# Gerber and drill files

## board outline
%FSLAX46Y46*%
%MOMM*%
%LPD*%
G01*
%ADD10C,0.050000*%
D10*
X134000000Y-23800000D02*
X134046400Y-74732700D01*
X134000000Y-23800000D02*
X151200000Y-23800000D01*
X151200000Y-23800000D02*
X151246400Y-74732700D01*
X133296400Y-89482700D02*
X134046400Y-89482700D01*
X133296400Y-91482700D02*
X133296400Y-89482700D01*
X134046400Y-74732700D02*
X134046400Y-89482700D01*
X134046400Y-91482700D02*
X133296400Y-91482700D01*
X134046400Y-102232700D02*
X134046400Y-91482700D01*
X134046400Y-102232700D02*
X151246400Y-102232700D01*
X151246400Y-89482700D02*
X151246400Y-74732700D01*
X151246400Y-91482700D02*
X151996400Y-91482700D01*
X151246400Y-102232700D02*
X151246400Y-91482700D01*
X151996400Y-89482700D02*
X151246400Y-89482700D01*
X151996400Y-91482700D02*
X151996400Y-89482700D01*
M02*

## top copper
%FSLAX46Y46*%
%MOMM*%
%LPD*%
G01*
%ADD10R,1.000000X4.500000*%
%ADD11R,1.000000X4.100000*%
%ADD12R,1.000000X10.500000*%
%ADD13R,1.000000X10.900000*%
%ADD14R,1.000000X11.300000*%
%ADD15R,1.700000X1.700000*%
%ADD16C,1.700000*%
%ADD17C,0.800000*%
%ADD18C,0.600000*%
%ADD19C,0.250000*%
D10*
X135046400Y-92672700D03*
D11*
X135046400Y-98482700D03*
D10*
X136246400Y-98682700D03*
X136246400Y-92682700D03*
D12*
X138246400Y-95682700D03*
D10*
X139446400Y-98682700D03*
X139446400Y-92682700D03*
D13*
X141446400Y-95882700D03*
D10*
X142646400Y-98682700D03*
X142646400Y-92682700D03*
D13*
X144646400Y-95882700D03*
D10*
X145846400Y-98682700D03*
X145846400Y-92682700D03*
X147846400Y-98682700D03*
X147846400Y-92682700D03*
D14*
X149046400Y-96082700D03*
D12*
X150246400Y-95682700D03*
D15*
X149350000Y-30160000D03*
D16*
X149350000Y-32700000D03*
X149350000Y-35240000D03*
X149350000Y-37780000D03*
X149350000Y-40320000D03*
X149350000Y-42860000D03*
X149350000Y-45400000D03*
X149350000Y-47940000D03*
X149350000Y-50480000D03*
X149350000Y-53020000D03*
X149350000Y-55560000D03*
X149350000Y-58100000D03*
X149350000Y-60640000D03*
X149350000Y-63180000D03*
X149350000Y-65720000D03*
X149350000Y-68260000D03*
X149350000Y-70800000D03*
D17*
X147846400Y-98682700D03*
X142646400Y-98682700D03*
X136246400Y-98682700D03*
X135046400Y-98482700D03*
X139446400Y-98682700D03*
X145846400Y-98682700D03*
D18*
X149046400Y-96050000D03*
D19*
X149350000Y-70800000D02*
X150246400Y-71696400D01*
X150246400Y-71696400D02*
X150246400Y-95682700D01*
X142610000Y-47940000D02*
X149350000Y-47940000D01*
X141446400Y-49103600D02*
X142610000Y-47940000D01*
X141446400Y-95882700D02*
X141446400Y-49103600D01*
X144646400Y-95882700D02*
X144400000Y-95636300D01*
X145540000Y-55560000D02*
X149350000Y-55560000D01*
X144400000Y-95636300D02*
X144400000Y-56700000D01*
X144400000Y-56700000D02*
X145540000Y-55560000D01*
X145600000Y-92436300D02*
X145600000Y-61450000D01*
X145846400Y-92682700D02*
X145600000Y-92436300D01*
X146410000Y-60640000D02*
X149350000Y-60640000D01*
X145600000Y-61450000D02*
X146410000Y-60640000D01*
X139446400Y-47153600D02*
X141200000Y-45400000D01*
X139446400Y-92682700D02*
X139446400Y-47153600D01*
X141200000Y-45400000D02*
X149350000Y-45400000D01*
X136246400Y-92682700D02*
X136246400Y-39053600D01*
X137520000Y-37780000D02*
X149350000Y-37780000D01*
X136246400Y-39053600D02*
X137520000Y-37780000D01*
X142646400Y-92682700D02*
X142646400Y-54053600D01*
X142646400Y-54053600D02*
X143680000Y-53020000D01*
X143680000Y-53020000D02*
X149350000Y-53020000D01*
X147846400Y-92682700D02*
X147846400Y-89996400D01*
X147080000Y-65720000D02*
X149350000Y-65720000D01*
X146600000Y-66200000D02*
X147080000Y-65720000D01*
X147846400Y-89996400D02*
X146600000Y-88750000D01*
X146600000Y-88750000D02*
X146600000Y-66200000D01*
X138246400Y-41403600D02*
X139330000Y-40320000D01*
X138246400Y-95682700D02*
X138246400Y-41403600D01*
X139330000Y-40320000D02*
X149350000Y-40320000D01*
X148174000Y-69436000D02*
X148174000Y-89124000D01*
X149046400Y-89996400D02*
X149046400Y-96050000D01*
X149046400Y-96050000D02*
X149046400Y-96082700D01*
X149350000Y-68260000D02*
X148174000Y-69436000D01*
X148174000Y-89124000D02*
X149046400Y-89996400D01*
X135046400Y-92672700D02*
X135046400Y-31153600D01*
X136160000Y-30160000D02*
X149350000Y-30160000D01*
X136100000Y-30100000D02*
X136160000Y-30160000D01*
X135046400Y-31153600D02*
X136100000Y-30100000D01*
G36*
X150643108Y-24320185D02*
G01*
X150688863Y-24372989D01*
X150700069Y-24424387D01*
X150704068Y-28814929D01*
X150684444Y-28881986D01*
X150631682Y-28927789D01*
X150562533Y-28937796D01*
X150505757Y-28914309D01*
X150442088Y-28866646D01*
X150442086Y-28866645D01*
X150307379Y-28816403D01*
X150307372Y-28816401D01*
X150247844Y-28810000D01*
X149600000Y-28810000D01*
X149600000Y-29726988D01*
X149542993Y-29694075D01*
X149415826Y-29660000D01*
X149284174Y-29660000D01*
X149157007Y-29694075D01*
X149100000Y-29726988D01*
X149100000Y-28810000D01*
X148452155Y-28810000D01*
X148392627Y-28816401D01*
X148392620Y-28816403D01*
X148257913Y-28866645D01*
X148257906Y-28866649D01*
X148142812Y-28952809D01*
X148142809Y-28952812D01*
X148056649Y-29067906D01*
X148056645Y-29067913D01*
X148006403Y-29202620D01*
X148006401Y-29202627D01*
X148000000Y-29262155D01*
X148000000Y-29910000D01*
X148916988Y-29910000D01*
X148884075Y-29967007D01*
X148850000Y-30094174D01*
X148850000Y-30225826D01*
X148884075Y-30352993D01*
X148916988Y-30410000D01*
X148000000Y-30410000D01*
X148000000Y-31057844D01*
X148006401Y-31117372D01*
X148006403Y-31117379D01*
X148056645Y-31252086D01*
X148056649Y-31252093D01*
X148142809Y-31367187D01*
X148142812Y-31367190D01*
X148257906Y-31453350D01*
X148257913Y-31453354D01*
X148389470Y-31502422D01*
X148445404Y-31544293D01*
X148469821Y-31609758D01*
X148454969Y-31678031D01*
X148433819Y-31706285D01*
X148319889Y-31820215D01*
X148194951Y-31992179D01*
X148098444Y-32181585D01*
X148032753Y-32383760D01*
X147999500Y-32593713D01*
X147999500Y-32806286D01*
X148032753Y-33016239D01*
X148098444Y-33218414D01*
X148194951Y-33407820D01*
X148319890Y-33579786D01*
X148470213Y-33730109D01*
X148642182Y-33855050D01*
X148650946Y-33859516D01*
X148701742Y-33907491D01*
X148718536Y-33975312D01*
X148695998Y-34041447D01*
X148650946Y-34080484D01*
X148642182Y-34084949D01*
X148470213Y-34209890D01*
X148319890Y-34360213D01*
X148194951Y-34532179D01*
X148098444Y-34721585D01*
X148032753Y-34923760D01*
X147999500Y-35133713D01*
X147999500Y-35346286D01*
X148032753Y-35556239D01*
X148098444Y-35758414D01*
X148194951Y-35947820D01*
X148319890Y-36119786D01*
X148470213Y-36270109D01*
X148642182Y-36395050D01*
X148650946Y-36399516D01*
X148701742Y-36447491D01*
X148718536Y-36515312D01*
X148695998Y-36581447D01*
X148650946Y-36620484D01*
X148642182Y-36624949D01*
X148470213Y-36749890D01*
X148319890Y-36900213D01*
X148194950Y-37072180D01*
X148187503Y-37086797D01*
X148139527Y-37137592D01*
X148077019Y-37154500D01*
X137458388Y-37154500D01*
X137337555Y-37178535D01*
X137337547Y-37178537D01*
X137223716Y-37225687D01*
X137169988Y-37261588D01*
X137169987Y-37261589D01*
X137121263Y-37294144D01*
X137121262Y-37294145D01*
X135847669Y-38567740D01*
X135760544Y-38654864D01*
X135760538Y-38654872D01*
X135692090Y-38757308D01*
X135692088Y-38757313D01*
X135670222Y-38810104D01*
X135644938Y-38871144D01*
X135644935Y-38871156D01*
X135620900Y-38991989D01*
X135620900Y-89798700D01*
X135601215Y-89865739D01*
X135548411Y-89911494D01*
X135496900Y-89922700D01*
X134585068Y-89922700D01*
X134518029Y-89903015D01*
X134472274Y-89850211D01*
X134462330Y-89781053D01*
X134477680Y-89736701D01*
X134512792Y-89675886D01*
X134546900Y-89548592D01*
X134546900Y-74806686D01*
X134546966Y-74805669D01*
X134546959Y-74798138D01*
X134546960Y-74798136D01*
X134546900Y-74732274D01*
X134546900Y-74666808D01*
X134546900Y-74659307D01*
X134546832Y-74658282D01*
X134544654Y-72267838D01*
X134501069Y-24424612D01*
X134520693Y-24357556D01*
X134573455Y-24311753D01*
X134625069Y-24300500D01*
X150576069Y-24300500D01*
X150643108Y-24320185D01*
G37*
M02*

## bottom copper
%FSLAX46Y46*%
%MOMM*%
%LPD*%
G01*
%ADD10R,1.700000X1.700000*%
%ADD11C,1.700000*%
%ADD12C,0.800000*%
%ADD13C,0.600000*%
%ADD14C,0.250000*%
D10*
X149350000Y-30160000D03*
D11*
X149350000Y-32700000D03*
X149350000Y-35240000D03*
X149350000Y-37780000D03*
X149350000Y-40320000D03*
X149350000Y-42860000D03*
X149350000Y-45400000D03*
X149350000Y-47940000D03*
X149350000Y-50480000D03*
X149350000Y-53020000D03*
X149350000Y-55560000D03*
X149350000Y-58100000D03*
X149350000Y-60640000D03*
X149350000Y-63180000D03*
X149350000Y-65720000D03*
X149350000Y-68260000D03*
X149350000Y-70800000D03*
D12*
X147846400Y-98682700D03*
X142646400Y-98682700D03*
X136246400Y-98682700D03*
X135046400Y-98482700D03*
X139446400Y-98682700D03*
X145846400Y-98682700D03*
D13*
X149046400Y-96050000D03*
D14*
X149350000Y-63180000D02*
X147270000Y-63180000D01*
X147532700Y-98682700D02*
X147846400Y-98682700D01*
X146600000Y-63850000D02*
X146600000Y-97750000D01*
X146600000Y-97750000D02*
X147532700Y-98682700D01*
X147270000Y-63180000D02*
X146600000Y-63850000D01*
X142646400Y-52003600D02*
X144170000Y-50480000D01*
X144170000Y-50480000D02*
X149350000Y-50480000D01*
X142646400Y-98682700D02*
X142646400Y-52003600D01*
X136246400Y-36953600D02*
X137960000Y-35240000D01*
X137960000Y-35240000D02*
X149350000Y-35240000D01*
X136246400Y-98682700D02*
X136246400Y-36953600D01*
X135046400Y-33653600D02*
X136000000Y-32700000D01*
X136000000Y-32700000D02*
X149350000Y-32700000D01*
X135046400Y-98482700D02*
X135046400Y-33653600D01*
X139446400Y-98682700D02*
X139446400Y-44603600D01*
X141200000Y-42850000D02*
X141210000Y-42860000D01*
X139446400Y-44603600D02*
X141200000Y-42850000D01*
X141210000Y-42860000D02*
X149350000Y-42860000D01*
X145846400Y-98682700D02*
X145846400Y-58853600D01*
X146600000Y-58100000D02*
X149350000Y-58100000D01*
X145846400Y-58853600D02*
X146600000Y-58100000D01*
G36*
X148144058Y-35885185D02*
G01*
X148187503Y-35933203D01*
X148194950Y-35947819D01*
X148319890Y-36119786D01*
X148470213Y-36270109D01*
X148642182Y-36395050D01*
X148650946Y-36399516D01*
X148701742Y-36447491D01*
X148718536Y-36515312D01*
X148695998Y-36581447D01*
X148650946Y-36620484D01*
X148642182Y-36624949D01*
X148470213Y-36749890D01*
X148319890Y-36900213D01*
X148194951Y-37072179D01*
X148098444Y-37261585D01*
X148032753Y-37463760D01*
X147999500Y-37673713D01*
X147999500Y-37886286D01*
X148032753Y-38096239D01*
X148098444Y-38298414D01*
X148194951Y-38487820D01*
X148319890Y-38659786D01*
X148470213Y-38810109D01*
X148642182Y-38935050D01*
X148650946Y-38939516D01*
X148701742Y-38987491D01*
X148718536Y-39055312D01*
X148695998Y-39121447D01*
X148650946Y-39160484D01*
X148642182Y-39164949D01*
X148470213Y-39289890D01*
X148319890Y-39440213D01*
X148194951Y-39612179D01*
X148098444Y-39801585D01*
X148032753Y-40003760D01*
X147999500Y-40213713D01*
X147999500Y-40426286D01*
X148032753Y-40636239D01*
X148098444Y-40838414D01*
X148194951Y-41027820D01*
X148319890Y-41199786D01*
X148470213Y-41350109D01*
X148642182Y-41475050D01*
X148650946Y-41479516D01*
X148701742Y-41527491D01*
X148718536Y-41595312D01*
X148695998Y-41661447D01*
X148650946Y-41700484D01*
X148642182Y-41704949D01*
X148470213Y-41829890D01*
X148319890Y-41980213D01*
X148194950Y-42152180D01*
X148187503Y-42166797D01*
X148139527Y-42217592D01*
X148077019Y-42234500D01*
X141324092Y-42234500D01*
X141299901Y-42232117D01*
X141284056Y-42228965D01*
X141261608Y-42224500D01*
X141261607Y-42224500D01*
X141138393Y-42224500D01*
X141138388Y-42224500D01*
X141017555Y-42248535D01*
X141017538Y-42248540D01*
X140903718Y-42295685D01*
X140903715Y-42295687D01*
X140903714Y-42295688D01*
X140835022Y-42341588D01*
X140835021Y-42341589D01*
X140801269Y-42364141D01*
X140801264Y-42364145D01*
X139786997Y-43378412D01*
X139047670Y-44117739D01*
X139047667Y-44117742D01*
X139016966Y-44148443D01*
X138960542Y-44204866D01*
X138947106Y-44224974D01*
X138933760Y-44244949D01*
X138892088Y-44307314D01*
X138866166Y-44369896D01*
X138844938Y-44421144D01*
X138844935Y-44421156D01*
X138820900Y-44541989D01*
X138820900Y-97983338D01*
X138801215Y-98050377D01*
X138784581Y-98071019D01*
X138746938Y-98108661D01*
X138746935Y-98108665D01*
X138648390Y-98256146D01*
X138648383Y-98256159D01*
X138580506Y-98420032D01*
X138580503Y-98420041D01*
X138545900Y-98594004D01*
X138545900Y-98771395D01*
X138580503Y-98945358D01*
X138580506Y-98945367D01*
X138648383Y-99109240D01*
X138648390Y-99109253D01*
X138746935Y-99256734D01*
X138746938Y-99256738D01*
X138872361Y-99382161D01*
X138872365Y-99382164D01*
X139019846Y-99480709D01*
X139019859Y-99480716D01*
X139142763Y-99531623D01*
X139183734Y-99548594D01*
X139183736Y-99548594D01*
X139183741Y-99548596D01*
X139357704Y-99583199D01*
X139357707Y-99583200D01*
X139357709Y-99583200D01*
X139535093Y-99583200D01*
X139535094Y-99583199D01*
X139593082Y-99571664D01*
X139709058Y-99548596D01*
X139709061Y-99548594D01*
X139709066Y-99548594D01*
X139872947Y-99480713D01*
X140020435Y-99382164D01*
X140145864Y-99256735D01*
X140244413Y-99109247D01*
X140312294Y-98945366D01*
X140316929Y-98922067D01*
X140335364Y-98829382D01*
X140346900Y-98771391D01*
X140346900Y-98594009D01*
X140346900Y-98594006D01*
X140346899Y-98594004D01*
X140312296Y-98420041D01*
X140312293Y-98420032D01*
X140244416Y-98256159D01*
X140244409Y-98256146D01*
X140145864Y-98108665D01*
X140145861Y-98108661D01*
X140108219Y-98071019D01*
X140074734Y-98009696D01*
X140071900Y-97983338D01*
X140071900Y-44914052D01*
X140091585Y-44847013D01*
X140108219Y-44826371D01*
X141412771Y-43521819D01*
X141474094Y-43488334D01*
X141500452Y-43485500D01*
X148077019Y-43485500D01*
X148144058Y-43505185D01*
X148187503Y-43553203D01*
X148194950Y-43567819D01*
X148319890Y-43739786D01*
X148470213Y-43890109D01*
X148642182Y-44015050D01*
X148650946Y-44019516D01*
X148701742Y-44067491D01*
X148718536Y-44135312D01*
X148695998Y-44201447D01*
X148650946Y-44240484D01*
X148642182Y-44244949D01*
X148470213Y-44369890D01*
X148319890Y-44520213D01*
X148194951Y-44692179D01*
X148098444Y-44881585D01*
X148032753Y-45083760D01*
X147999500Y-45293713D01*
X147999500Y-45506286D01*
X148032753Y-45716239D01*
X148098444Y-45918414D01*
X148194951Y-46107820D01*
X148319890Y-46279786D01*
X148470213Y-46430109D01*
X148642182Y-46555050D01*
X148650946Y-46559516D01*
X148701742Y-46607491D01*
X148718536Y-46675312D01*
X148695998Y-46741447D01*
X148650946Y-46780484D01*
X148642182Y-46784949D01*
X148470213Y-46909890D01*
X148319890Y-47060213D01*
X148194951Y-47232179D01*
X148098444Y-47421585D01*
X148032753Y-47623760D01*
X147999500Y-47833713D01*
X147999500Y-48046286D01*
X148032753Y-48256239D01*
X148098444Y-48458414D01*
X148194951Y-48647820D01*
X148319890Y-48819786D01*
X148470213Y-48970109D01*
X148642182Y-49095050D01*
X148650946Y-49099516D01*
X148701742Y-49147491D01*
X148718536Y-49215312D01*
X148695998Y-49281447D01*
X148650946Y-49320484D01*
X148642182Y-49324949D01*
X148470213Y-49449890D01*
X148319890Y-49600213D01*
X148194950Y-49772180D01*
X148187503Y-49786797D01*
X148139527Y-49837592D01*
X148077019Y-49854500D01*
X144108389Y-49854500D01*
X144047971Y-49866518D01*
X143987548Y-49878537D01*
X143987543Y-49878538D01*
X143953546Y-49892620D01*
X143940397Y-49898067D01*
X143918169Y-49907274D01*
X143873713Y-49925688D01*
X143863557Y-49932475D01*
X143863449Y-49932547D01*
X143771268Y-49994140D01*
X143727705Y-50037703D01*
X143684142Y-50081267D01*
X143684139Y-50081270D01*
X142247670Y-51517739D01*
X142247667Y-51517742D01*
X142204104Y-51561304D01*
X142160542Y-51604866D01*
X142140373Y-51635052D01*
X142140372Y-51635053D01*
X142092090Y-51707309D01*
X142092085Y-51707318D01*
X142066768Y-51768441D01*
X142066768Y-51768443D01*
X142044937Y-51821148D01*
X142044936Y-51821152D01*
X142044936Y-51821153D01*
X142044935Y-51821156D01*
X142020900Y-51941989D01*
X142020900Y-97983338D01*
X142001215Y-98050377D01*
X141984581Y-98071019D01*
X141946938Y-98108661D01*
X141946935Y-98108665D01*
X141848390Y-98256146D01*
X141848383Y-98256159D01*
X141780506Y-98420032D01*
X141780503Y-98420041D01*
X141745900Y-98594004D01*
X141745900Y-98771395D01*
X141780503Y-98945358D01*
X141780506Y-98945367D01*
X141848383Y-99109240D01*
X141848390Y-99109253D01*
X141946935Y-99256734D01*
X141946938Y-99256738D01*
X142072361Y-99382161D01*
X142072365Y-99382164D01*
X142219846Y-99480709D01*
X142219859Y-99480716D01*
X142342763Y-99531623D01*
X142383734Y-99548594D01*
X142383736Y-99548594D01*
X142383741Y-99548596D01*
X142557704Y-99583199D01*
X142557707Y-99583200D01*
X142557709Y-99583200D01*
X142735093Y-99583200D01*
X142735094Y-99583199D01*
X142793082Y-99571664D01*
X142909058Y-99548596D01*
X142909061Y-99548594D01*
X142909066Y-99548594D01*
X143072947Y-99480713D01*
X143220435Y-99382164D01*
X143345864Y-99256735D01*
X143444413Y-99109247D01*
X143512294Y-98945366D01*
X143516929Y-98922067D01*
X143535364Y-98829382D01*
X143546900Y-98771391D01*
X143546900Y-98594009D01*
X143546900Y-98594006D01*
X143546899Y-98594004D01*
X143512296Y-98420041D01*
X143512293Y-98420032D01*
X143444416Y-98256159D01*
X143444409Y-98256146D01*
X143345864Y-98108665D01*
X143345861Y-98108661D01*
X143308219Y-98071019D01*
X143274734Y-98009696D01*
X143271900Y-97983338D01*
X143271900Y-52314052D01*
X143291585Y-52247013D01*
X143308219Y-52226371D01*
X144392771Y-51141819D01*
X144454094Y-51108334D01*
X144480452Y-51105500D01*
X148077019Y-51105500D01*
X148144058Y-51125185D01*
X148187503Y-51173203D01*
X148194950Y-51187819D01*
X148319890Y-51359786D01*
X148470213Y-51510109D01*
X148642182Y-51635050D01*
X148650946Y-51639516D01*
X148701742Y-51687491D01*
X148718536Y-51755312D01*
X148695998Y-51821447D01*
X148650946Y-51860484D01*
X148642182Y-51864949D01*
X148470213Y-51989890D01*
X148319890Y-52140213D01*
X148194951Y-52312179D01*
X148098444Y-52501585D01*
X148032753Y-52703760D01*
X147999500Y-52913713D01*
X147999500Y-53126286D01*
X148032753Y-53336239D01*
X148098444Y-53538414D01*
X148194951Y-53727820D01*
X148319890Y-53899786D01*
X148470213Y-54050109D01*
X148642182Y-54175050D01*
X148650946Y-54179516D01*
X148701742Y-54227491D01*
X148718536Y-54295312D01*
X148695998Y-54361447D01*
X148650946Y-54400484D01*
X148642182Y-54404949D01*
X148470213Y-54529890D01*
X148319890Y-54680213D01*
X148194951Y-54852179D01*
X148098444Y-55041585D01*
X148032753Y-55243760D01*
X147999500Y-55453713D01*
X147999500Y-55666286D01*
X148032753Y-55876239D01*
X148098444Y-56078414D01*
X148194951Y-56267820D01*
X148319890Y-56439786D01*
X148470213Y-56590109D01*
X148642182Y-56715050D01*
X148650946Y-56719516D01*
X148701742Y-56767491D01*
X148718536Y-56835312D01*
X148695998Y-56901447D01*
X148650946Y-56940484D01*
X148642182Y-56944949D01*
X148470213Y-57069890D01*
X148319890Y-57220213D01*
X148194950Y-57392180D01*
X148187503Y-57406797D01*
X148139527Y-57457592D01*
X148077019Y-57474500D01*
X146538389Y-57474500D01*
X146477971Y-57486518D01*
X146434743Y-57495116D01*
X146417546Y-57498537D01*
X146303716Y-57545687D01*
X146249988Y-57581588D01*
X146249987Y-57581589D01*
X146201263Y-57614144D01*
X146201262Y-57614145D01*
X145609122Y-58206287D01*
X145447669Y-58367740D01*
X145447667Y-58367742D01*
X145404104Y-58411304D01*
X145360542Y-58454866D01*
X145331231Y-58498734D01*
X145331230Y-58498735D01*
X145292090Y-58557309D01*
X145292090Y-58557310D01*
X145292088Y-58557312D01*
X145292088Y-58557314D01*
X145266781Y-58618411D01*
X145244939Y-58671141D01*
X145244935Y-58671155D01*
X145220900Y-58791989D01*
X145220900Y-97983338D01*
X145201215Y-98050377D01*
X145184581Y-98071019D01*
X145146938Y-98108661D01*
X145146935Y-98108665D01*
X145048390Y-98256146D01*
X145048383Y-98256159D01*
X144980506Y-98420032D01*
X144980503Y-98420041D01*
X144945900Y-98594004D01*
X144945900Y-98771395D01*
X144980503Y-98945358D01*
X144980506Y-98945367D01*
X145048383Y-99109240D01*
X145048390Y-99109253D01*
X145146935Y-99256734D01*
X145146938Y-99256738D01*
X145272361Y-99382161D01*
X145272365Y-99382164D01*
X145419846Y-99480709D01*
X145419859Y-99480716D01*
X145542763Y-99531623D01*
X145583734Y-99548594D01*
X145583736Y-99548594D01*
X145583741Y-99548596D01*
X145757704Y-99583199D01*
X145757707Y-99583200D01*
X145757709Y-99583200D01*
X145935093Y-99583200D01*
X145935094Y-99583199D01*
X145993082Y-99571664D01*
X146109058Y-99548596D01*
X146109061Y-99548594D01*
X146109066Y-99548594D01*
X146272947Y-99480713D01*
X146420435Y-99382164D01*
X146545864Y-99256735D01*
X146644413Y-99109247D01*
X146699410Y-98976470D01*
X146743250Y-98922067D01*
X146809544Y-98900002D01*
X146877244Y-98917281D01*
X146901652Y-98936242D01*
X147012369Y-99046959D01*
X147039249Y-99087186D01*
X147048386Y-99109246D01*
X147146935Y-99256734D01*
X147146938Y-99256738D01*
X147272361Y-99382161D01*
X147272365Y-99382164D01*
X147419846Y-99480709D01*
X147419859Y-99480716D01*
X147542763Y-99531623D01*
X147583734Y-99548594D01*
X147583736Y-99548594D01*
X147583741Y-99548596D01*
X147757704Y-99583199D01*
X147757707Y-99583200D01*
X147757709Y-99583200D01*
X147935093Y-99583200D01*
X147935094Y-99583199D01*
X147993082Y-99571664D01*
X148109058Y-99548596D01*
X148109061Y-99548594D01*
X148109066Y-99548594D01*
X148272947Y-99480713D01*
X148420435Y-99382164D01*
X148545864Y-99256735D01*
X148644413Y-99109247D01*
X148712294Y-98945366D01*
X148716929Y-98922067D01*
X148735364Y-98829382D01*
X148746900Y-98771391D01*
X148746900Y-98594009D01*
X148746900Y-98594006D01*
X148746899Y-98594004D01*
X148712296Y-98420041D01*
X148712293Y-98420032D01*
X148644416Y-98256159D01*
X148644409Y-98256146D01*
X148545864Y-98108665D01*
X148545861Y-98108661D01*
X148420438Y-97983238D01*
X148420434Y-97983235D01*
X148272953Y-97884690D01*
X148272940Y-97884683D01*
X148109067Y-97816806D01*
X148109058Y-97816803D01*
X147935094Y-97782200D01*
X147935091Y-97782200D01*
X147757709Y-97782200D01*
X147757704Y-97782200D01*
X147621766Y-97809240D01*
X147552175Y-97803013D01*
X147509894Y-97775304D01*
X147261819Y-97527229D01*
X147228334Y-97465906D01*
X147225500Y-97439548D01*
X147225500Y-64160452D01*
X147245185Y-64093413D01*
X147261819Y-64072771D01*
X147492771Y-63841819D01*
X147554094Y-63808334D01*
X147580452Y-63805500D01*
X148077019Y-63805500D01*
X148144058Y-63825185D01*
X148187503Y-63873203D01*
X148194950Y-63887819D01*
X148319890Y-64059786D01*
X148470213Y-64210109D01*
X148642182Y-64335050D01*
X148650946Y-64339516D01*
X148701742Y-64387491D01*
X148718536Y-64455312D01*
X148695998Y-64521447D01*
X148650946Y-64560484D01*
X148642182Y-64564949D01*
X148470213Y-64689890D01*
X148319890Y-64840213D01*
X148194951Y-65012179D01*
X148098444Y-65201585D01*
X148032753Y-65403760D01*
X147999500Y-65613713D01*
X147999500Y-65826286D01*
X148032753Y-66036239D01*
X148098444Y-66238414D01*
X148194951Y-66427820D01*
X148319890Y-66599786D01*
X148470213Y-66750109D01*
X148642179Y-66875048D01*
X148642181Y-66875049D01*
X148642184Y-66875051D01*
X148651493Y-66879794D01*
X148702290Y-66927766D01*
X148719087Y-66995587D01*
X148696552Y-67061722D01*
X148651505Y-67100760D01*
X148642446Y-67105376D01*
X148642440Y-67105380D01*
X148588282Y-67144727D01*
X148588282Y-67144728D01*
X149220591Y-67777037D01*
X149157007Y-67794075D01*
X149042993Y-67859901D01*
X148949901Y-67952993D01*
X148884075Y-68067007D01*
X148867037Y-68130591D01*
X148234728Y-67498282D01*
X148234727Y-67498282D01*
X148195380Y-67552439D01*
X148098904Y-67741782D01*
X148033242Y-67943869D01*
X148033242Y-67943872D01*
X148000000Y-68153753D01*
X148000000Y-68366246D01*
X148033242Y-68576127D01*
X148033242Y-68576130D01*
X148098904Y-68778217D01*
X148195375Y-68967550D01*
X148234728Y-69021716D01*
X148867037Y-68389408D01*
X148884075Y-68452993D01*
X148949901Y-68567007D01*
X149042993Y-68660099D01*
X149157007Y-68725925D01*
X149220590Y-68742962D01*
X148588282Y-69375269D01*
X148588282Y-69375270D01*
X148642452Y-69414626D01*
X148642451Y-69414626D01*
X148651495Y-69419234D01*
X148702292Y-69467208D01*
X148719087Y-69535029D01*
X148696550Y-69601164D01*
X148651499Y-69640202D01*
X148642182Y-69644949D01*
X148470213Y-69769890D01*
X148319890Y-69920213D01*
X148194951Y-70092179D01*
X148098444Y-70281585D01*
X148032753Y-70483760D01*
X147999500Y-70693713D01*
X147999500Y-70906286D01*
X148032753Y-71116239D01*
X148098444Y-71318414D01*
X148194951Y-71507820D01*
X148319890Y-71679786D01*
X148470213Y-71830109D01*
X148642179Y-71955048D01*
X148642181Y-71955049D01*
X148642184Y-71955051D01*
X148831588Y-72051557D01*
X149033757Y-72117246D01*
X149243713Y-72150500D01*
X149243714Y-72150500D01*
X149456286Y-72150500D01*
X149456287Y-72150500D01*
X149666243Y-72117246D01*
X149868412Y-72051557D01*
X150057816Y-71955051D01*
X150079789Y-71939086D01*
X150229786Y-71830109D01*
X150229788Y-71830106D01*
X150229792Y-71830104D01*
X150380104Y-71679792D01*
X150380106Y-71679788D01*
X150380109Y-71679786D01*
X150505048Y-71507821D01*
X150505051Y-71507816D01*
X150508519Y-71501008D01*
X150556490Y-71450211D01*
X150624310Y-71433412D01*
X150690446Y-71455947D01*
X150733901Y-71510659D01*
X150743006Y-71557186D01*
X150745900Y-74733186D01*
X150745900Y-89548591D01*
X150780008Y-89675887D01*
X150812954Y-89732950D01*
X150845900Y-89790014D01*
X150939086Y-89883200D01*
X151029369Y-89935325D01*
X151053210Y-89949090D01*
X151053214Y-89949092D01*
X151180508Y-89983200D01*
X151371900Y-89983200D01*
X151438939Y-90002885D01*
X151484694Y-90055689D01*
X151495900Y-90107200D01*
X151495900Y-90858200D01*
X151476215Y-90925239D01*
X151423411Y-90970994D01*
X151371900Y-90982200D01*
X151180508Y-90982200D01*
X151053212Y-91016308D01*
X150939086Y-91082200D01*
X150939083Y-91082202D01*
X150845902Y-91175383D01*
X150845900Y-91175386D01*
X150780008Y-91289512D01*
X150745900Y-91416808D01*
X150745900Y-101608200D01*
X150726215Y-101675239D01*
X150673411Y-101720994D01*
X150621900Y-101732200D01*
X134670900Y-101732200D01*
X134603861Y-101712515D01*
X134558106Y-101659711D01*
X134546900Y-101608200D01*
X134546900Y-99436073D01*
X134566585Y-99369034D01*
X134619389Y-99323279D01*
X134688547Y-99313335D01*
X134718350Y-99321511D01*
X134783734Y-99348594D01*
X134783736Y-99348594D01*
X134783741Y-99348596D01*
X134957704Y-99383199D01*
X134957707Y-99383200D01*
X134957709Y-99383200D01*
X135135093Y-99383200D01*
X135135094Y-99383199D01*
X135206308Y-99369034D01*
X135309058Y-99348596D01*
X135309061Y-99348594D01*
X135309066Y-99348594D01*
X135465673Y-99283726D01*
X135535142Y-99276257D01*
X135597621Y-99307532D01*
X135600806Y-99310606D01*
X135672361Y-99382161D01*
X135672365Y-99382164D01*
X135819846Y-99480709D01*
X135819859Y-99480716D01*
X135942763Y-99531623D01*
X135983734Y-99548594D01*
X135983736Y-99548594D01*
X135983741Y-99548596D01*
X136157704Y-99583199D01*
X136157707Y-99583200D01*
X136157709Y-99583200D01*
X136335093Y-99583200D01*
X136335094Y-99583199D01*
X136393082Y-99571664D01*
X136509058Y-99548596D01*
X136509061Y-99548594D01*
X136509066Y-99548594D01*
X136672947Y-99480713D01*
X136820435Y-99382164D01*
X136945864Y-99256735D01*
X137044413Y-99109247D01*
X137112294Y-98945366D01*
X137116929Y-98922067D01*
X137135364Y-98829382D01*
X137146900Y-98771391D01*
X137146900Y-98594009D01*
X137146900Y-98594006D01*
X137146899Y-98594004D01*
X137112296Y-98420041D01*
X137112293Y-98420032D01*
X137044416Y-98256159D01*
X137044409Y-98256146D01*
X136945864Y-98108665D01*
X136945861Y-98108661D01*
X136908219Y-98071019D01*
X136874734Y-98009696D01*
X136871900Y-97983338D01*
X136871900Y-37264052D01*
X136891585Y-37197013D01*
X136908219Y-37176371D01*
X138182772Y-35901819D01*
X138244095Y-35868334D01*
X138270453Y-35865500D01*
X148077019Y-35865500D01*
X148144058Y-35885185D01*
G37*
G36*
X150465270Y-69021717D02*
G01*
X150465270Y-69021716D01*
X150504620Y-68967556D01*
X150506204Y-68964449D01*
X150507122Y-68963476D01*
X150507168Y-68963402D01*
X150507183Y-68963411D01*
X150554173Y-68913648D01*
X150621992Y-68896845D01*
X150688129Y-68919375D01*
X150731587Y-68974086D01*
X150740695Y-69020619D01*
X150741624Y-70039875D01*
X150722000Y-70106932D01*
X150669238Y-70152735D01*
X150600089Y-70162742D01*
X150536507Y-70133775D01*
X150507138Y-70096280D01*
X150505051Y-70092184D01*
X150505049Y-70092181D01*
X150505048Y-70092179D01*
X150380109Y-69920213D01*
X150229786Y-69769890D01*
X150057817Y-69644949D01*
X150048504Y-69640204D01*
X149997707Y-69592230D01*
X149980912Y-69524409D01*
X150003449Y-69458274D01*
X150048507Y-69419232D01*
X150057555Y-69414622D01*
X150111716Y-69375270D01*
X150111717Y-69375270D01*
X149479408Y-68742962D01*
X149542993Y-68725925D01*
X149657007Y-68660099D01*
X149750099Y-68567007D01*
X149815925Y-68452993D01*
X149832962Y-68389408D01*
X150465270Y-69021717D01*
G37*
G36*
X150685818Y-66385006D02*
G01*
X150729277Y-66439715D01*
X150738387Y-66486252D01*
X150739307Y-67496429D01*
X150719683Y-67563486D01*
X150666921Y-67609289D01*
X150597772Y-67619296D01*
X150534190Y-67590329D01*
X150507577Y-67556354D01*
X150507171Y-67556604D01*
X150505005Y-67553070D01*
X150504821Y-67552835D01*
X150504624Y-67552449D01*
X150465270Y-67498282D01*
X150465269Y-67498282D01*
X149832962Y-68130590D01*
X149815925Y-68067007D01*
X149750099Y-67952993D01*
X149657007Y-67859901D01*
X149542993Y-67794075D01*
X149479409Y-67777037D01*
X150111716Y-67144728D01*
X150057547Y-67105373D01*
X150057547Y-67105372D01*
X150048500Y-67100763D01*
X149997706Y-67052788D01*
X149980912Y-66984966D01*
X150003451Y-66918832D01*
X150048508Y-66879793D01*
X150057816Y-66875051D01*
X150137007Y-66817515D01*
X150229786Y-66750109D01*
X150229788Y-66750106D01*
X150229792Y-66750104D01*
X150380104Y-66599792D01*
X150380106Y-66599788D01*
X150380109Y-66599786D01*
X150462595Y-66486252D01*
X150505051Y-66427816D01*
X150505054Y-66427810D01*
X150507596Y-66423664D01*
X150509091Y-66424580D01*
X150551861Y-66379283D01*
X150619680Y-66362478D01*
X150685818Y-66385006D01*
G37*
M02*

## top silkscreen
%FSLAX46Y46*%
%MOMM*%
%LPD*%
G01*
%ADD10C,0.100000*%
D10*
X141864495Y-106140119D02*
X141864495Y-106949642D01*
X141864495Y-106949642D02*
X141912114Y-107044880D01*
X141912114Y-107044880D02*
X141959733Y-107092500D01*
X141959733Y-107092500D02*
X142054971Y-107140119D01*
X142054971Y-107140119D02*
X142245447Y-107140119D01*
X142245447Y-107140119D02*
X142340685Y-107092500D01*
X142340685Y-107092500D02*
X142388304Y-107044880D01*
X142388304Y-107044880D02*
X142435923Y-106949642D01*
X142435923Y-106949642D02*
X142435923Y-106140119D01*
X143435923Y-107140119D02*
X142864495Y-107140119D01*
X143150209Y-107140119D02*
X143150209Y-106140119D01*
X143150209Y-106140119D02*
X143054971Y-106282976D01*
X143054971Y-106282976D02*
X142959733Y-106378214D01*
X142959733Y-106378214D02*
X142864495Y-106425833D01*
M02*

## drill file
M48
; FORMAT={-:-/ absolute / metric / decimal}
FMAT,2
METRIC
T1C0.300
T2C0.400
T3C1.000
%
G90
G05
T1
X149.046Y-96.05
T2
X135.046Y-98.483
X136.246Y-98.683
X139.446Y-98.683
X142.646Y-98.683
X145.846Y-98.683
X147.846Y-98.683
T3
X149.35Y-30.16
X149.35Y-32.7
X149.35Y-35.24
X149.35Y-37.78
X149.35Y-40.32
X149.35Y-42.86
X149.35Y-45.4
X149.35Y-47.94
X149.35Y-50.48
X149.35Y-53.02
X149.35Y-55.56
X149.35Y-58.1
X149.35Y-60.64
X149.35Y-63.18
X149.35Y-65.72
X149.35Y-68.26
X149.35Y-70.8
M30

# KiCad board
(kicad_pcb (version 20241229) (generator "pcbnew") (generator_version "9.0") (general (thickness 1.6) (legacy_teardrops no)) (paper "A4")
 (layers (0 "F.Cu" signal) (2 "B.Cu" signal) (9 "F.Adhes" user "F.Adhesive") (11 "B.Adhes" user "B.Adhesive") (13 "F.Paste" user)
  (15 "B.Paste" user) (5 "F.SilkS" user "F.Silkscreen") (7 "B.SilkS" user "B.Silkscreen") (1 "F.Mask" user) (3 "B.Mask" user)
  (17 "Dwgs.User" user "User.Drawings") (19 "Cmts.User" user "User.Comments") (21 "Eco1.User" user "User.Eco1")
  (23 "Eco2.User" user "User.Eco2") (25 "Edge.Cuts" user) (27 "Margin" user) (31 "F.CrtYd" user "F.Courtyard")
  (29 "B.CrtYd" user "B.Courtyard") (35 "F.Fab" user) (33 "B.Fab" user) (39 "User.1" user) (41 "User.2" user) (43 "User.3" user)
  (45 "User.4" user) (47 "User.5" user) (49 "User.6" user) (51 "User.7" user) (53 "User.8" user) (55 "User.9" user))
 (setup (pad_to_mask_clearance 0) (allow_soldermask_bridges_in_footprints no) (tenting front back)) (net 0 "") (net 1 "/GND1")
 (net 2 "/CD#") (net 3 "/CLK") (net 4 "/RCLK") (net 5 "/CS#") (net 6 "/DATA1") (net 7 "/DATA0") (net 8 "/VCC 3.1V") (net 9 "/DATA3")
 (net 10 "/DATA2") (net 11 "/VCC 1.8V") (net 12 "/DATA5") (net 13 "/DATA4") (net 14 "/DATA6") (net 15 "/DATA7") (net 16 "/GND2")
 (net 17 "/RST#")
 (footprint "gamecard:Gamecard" (layer "F.Cu") (at 142.6464 102.2327)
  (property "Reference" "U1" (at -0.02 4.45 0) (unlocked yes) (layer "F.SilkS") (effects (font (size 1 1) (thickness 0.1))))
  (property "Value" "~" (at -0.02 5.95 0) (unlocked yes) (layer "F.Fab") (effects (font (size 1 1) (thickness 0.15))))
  (fp_line (start -9.35 -12.75) (end -8.6 -12.75) (stroke (width 0.05) (type default)) (layer "Edge.Cuts"))
  (fp_line (start -9.35 -10.75) (end -9.35 -12.75) (stroke (width 0.05) (type default)) (layer "Edge.Cuts"))
  (fp_line (start -8.6 -27.5) (end -8.6 -12.75) (stroke (width 0.05) (type default)) (layer "Edge.Cuts"))
  (fp_line (start -8.6 -10.75) (end -9.35 -10.75) (stroke (width 0.05) (type default)) (layer "Edge.Cuts"))
  (fp_line (start -8.6 0) (end -8.6 -10.75) (stroke (width 0.05) (type default)) (layer "Edge.Cuts"))
  (fp_line (start -8.6 0) (end 8.6 0) (stroke (width 0.05) (type default)) (layer "Edge.Cuts"))
  (fp_line (start 8.6 -12.75) (end 8.6 -27.5) (stroke (width 0.05) (type default)) (layer "Edge.Cuts"))
  (fp_line (start 8.6 -10.75) (end 9.35 -10.75) (stroke (width 0.05) (type default)) (layer "Edge.Cuts"))
  (fp_line (start 8.6 0) (end 8.6 -10.75) (stroke (width 0.05) (type default)) (layer "Edge.Cuts"))
  (fp_line (start 9.35 -12.75) (end 8.6 -12.75) (stroke (width 0.05) (type default)) (layer "Edge.Cuts"))
  (fp_line (start 9.35 -10.75) (end 9.35 -12.75) (stroke (width 0.05) (type default)) (layer "Edge.Cuts"))
  (pad "1" smd rect (at -7.6 -9.56) (size 1 4.5) (layers "F.Cu" "F.Mask" "F.Paste") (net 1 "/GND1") (thermal_bridge_angle 45))
  (pad "2" smd rect (at -7.6 -3.75) (size 1 4.1) (layers "F.Cu" "F.Mask" "F.Paste") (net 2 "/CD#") (thermal_bridge_angle 45))
  (pad "3" smd rect (at -6.4 -3.55) (size 1 4.5) (layers "F.Cu" "F.Mask" "F.Paste") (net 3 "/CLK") (thermal_bridge_angle 45))
  (pad "4" smd rect (at -6.4 -9.55) (size 1 4.5) (layers "F.Cu" "F.Mask" "F.Paste") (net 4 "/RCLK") (thermal_bridge_angle 45))
  (pad "5" smd rect (at -4.4 -6.55) (size 1 10.5) (layers "F.Cu" "F.Mask" "F.Paste") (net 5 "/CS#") (thermal_bridge_angle 45))
  (pad "6" smd rect (at -3.2 -3.55) (size 1 4.5) (layers "F.Cu" "F.Mask" "F.Paste") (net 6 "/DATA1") (thermal_bridge_angle 45))
  (pad "7" smd rect (at -3.2 -9.55) (size 1 4.5) (layers "F.Cu" "F.Mask" "F.Paste") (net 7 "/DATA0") (thermal_bridge_angle 45))
  (pad "8" smd rect (at -1.2 -6.35) (size 1 10.9) (layers "F.Cu" "F.Mask" "F.Paste") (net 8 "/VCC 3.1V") (thermal_bridge_angle 45))
  (pad "9" smd rect (at 0 -3.55) (size 1 4.5) (layers "F.Cu" "F.Mask" "F.Paste") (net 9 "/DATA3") (thermal_bridge_angle 45))
  (pad "10" smd rect (at 0 -9.55) (size 1 4.5) (layers "F.Cu" "F.Mask" "F.Paste") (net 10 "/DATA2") (thermal_bridge_angle 45))
  (pad "11" smd rect (at 2 -6.35) (size 1 10.9) (layers "F.Cu" "F.Mask" "F.Paste") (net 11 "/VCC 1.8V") (thermal_bridge_angle 45))
  (pad "12" smd rect (at 3.2 -3.55) (size 1 4.5) (layers "F.Cu" "F.Mask" "F.Paste") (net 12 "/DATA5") (thermal_bridge_angle 45))
  (pad "13" smd rect (at 3.2 -9.55) (size 1 4.5) (layers "F.Cu" "F.Mask" "F.Paste") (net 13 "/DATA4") (thermal_bridge_angle 45))
  (pad "14" smd rect (at 5.2 -3.55) (size 1 4.5) (layers "F.Cu" "F.Mask" "F.Paste") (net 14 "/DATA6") (thermal_bridge_angle 45))
  (pad "15" smd rect (at 5.2 -9.55) (size 1 4.5) (layers "F.Cu" "F.Mask" "F.Paste") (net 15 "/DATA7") (thermal_bridge_angle 45))
  (pad "16" smd rect (at 6.4 -6.15) (size 1 11.3) (layers "F.Cu" "F.Mask" "F.Paste") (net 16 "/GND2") (thermal_bridge_angle 45))
  (pad "17" smd rect (at 7.6 -6.55) (size 1 10.5) (layers "F.Cu" "F.Mask" "F.Paste") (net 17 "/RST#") (thermal_bridge_angle 45))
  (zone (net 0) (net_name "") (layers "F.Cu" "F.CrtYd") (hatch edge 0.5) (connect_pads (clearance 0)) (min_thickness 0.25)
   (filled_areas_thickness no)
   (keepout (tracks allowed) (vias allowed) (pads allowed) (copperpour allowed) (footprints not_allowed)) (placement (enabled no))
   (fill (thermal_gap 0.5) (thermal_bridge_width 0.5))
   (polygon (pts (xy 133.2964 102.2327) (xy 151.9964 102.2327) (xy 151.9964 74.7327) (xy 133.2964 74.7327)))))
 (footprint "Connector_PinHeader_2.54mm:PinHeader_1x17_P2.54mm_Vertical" (layer "B.Cu") (at 149.35 30.16 180)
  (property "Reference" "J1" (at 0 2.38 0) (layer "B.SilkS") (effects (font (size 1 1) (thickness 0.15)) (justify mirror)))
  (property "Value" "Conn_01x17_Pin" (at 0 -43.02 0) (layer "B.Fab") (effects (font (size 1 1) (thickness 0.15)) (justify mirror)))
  (pad "1" thru_hole rect (at 0 0 180) (size 1.7 1.7) (drill 1) (layers "*.Cu" "*.Mask") (remove_unused_layers no) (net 1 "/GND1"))
  (pad "2" thru_hole circle (at 0 -2.54 180) (size 1.7 1.7) (drill 1) (layers "*.Cu" "*.Mask") (remove_unused_layers no) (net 2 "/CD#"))
  (pad "3" thru_hole circle (at 0 -5.08 180) (size 1.7 1.7) (drill 1) (layers "*.Cu" "*.Mask") (remove_unused_layers no) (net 3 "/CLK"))
  (pad "4" thru_hole circle (at 0 -7.62 180) (size 1.7 1.7) (drill 1) (layers "*.Cu" "*.Mask") (remove_unused_layers no) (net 4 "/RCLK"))
  (pad "5" thru_hole circle (at 0 -10.16 180) (size 1.7 1.7) (drill 1) (layers "*.Cu" "*.Mask") (remove_unused_layers no) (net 5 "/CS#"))
  (pad "6" thru_hole circle (at 0 -12.7 180) (size 1.7 1.7) (drill 1) (layers "*.Cu" "*.Mask") (remove_unused_layers no) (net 6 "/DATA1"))
  (pad "7" thru_hole circle (at 0 -15.24 180) (size 1.7 1.7) (drill 1) (layers "*.Cu" "*.Mask") (remove_unused_layers no) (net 7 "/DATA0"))
  (pad "8" thru_hole circle (at 0 -17.78 180) (size 1.7 1.7) (drill 1) (layers "*.Cu" "*.Mask") (remove_unused_layers no)
   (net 8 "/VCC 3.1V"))
  (pad "9" thru_hole circle (at 0 -20.32 180) (size 1.7 1.7) (drill 1) (layers "*.Cu" "*.Mask") (remove_unused_layers no) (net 9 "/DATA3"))
  (pad "10" thru_hole circle (at 0 -22.86 180) (size 1.7 1.7) (drill 1) (layers "*.Cu" "*.Mask") (remove_unused_layers no) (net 10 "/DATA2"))
  (pad "11" thru_hole circle (at 0 -25.4 180) (size 1.7 1.7) (drill 1) (layers "*.Cu" "*.Mask") (remove_unused_layers no)
   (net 11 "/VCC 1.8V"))
  (pad "12" thru_hole circle (at 0 -27.94 180) (size 1.7 1.7) (drill 1) (layers "*.Cu" "*.Mask") (remove_unused_layers no) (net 12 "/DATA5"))
  (pad "13" thru_hole circle (at 0 -30.48 180) (size 1.7 1.7) (drill 1) (layers "*.Cu" "*.Mask") (remove_unused_layers no) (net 13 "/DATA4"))
  (pad "14" thru_hole circle (at 0 -33.02 180) (size 1.7 1.7) (drill 1) (layers "*.Cu" "*.Mask") (remove_unused_layers no) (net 14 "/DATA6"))
  (pad "15" thru_hole circle (at 0 -35.56 180) (size 1.7 1.7) (drill 1) (layers "*.Cu" "*.Mask") (remove_unused_layers no) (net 15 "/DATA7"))
  (pad "16" thru_hole circle (at 0 -38.1 180) (size 1.7 1.7) (drill 1) (layers "*.Cu" "*.Mask") (remove_unused_layers no) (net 16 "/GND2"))
  (pad "17" thru_hole circle (at 0 -40.64 180) (size 1.7 1.7) (drill 1) (layers "*.Cu" "*.Mask") (remove_unused_layers no) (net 17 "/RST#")))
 (gr_line (start 134 23.8) (end 134.0464 74.7327) (stroke (width 0.05) (type default)) (layer "Edge.Cuts"))
 (gr_line (start 134 23.8) (end 151.2 23.8) (stroke (width 0.05) (type default)) (layer "Edge.Cuts"))
 (gr_line (start 151.2 23.8) (end 151.2464 74.7327) (stroke (width 0.05) (type default)) (layer "Edge.Cuts"))
 (segment (start 149.35 70.8) (end 150.2464 71.6964) (width 0.25) (layer "F.Cu") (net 17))
 (segment (start 150.2464 71.6964) (end 150.2464 95.6827) (width 0.25) (layer "F.Cu") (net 17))
 (segment (start 142.61 47.94) (end 149.35 47.94) (width 0.25) (layer "F.Cu") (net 8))
 (segment (start 141.4464 49.1036) (end 142.61 47.94) (width 0.25) (layer "F.Cu") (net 8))
 (segment (start 141.4464 95.8827) (end 141.4464 49.1036) (width 0.25) (layer "F.Cu") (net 8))
 (segment (start 144.6464 95.8827) (end 144.4 95.6363) (width 0.25) (layer "F.Cu") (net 11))
 (segment (start 145.54 55.56) (end 149.35 55.56) (width 0.25) (layer "F.Cu") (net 11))
 (segment (start 144.4 95.6363) (end 144.4 56.7) (width 0.25) (layer "F.Cu") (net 11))
 (segment (start 144.4 56.7) (end 145.54 55.56) (width 0.25) (layer "F.Cu") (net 11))
 (segment (start 145.6 92.4363) (end 145.6 61.45) (width 0.25) (layer "F.Cu") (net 13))
 (segment (start 145.8464 92.6827) (end 145.6 92.4363) (width 0.25) (layer "F.Cu") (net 13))
 (segment (start 146.41 60.64) (end 149.35 60.64) (width 0.25) (layer "F.Cu") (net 13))
 (segment (start 145.6 61.45) (end 146.41 60.64) (width 0.25) (layer "F.Cu") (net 13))
 (segment (start 139.4464 47.1536) (end 141.2 45.4) (width 0.25) (layer "F.Cu") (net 7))
 (segment (start 139.4464 92.6827) (end 139.4464 47.1536) (width 0.25) (layer "F.Cu") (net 7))
 (segment (start 141.2 45.4) (end 149.35 45.4) (width 0.25) (layer "F.Cu") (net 7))
 (segment (start 136.2464 92.6827) (end 136.2464 39.0536) (width 0.25) (layer "F.Cu") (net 4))
 (segment (start 137.52 37.78) (end 149.35 37.78) (width 0.25) (layer "F.Cu") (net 4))
 (segment (start 136.2464 39.0536) (end 137.52 37.78) (width 0.25) (layer "F.Cu") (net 4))
 (segment (start 142.6464 92.6827) (end 142.6464 54.0536) (width 0.25) (layer "F.Cu") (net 10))
 (segment (start 142.6464 54.0536) (end 143.68 53.02) (width 0.25) (layer "F.Cu") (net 10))
 (segment (start 143.68 53.02) (end 149.35 53.02) (width 0.25) (layer "F.Cu") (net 10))
 (via (at 147.8464 98.6827) (size 0.8) (drill 0.4) (layers "F.Cu" "B.Cu") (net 14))
 (segment (start 149.35 63.18) (end 147.27 63.18) (width 0.25) (layer "B.Cu") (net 14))
 (segment (start 147.5327 98.6827) (end 147.8464 98.6827) (width 0.25) (layer "B.Cu") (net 14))
 (segment (start 146.6 63.85) (end 146.6 97.75) (width 0.25) (layer "B.Cu") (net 14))
 (segment (start 146.6 97.75) (end 147.5327 98.6827) (width 0.25) (layer "B.Cu") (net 14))
 (segment (start 147.27 63.18) (end 146.6 63.85) (width 0.25) (layer "B.Cu") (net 14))
 (segment (start 147.8464 92.6827) (end 147.8464 89.9964) (width 0.25) (layer "F.Cu") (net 15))
 (segment (start 147.08 65.72) (end 149.35 65.72) (width 0.25) (layer "F.Cu") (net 15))
 (segment (start 146.6 66.2) (end 147.08 65.72) (width 0.25) (layer "F.Cu") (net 15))
 (segment (start 147.8464 89.9964) (end 146.6 88.75) (width 0.25) (layer "F.Cu") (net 15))
 (segment (start 146.6 88.75) (end 146.6 66.2) (width 0.25) (layer "F.Cu") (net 15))
 (via (at 142.6464 98.6827) (size 0.8) (drill 0.4) (layers "F.Cu" "B.Cu") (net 9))
 (segment (start 142.6464 52.0036) (end 144.17 50.48) (width 0.25) (layer "B.Cu") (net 9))
 (segment (start 144.17 50.48) (end 149.35 50.48) (width 0.25) (layer "B.Cu") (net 9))
 (segment (start 142.6464 98.6827) (end 142.6464 52.0036) (width 0.25) (layer "B.Cu") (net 9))
 (via (at 136.2464 98.6827) (size 0.8) (drill 0.4) (layers "F.Cu" "B.Cu") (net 3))
 (segment (start 136.2464 36.9536) (end 137.96 35.24) (width 0.25) (layer "B.Cu") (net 3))
 (segment (start 137.96 35.24) (end 149.35 35.24) (width 0.25) (layer "B.Cu") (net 3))
 (segment (start 136.2464 98.6827) (end 136.2464 36.9536) (width 0.25) (layer "B.Cu") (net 3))
 (via (at 135.0464 98.4827) (size 0.8) (drill 0.4) (layers "F.Cu" "B.Cu") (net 2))
 (segment (start 135.0464 33.6536) (end 136 32.7) (width 0.25) (layer "B.Cu") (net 2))
 (segment (start 136 32.7) (end 149.35 32.7) (width 0.25) (layer "B.Cu") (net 2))
 (segment (start 135.0464 98.4827) (end 135.0464 33.6536) (width 0.25) (layer "B.Cu") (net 2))
 (via (at 139.4464 98.6827) (size 0.8) (drill 0.4) (layers "F.Cu" "B.Cu") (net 6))
 (segment (start 139.4464 98.6827) (end 139.4464 44.6036) (width 0.25) (layer "B.Cu") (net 6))
 (segment (start 141.2 42.85) (end 141.21 42.86) (width 0.25) (layer "B.Cu") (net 6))
 (segment (start 139.4464 44.6036) (end 141.2 42.85) (width 0.25) (layer "B.Cu") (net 6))
 (segment (start 141.21 42.86) (end 149.35 42.86) (width 0.25) (layer "B.Cu") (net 6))
 (segment (start 138.2464 41.4036) (end 139.33 40.32) (width 0.25) (layer "F.Cu") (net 5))
 (segment (start 138.2464 95.6827) (end 138.2464 41.4036) (width 0.25) (layer "F.Cu") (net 5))
 (segment (start 139.33 40.32) (end 149.35 40.32) (width 0.25) (layer "F.Cu") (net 5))
 (via (at 145.8464 98.6827) (size 0.8) (drill 0.4) (layers "F.Cu" "B.Cu") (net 12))
 (segment (start 145.8464 98.6827) (end 145.8464 58.8536) (width 0.25) (layer "B.Cu") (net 12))
 (segment (start 146.6 58.1) (end 149.35 58.1) (width 0.25) (layer "B.Cu") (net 12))
 (segment (start 145.8464 58.8536) (end 146.6 58.1) (width 0.25) (layer "B.Cu") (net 12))
 (segment (start 148.174 69.436) (end 148.174 89.124) (width 0.25) (layer "F.Cu") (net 16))
 (segment (start 149.0464 89.9964) (end 149.0464 96.05) (width 0.25) (layer "F.Cu") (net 16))
 (segment (start 149.0464 96.05) (end 149.0464 96.0827) (width 0.25) (layer "F.Cu") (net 16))
 (segment (start 149.35 68.26) (end 148.174 69.436) (width 0.25) (layer "F.Cu") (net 16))
 (segment (start 148.174 89.124) (end 149.0464 89.9964) (width 0.25) (layer "F.Cu") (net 16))
 (via (at 149.0464 96.05) (size 0.6) (drill 0.3) (layers "F.Cu" "B.Cu") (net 16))
 (segment (start 135.0464 92.6727) (end 135.0464 31.1536) (width 0.25) (layer "F.Cu") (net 1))
 (segment (start 136.16 30.16) (end 149.35 30.16) (width 0.25) (layer "F.Cu") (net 1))
 (segment (start 136.1 30.1) (end 136.16 30.16) (width 0.25) (layer "F.Cu") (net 1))
 (segment (start 135.0464 31.1536) (end 136.1 30.1) (width 0.25) (layer "F.Cu") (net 1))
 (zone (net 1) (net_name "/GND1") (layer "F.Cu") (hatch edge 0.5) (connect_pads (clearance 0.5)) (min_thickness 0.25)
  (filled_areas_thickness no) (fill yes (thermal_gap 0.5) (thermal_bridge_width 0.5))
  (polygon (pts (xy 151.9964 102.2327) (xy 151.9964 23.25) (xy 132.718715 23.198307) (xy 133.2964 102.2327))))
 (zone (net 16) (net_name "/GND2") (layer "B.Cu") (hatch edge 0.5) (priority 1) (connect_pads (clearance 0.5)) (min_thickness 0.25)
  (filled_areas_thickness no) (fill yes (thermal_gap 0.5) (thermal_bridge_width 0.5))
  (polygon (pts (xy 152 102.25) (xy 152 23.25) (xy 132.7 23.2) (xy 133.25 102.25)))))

